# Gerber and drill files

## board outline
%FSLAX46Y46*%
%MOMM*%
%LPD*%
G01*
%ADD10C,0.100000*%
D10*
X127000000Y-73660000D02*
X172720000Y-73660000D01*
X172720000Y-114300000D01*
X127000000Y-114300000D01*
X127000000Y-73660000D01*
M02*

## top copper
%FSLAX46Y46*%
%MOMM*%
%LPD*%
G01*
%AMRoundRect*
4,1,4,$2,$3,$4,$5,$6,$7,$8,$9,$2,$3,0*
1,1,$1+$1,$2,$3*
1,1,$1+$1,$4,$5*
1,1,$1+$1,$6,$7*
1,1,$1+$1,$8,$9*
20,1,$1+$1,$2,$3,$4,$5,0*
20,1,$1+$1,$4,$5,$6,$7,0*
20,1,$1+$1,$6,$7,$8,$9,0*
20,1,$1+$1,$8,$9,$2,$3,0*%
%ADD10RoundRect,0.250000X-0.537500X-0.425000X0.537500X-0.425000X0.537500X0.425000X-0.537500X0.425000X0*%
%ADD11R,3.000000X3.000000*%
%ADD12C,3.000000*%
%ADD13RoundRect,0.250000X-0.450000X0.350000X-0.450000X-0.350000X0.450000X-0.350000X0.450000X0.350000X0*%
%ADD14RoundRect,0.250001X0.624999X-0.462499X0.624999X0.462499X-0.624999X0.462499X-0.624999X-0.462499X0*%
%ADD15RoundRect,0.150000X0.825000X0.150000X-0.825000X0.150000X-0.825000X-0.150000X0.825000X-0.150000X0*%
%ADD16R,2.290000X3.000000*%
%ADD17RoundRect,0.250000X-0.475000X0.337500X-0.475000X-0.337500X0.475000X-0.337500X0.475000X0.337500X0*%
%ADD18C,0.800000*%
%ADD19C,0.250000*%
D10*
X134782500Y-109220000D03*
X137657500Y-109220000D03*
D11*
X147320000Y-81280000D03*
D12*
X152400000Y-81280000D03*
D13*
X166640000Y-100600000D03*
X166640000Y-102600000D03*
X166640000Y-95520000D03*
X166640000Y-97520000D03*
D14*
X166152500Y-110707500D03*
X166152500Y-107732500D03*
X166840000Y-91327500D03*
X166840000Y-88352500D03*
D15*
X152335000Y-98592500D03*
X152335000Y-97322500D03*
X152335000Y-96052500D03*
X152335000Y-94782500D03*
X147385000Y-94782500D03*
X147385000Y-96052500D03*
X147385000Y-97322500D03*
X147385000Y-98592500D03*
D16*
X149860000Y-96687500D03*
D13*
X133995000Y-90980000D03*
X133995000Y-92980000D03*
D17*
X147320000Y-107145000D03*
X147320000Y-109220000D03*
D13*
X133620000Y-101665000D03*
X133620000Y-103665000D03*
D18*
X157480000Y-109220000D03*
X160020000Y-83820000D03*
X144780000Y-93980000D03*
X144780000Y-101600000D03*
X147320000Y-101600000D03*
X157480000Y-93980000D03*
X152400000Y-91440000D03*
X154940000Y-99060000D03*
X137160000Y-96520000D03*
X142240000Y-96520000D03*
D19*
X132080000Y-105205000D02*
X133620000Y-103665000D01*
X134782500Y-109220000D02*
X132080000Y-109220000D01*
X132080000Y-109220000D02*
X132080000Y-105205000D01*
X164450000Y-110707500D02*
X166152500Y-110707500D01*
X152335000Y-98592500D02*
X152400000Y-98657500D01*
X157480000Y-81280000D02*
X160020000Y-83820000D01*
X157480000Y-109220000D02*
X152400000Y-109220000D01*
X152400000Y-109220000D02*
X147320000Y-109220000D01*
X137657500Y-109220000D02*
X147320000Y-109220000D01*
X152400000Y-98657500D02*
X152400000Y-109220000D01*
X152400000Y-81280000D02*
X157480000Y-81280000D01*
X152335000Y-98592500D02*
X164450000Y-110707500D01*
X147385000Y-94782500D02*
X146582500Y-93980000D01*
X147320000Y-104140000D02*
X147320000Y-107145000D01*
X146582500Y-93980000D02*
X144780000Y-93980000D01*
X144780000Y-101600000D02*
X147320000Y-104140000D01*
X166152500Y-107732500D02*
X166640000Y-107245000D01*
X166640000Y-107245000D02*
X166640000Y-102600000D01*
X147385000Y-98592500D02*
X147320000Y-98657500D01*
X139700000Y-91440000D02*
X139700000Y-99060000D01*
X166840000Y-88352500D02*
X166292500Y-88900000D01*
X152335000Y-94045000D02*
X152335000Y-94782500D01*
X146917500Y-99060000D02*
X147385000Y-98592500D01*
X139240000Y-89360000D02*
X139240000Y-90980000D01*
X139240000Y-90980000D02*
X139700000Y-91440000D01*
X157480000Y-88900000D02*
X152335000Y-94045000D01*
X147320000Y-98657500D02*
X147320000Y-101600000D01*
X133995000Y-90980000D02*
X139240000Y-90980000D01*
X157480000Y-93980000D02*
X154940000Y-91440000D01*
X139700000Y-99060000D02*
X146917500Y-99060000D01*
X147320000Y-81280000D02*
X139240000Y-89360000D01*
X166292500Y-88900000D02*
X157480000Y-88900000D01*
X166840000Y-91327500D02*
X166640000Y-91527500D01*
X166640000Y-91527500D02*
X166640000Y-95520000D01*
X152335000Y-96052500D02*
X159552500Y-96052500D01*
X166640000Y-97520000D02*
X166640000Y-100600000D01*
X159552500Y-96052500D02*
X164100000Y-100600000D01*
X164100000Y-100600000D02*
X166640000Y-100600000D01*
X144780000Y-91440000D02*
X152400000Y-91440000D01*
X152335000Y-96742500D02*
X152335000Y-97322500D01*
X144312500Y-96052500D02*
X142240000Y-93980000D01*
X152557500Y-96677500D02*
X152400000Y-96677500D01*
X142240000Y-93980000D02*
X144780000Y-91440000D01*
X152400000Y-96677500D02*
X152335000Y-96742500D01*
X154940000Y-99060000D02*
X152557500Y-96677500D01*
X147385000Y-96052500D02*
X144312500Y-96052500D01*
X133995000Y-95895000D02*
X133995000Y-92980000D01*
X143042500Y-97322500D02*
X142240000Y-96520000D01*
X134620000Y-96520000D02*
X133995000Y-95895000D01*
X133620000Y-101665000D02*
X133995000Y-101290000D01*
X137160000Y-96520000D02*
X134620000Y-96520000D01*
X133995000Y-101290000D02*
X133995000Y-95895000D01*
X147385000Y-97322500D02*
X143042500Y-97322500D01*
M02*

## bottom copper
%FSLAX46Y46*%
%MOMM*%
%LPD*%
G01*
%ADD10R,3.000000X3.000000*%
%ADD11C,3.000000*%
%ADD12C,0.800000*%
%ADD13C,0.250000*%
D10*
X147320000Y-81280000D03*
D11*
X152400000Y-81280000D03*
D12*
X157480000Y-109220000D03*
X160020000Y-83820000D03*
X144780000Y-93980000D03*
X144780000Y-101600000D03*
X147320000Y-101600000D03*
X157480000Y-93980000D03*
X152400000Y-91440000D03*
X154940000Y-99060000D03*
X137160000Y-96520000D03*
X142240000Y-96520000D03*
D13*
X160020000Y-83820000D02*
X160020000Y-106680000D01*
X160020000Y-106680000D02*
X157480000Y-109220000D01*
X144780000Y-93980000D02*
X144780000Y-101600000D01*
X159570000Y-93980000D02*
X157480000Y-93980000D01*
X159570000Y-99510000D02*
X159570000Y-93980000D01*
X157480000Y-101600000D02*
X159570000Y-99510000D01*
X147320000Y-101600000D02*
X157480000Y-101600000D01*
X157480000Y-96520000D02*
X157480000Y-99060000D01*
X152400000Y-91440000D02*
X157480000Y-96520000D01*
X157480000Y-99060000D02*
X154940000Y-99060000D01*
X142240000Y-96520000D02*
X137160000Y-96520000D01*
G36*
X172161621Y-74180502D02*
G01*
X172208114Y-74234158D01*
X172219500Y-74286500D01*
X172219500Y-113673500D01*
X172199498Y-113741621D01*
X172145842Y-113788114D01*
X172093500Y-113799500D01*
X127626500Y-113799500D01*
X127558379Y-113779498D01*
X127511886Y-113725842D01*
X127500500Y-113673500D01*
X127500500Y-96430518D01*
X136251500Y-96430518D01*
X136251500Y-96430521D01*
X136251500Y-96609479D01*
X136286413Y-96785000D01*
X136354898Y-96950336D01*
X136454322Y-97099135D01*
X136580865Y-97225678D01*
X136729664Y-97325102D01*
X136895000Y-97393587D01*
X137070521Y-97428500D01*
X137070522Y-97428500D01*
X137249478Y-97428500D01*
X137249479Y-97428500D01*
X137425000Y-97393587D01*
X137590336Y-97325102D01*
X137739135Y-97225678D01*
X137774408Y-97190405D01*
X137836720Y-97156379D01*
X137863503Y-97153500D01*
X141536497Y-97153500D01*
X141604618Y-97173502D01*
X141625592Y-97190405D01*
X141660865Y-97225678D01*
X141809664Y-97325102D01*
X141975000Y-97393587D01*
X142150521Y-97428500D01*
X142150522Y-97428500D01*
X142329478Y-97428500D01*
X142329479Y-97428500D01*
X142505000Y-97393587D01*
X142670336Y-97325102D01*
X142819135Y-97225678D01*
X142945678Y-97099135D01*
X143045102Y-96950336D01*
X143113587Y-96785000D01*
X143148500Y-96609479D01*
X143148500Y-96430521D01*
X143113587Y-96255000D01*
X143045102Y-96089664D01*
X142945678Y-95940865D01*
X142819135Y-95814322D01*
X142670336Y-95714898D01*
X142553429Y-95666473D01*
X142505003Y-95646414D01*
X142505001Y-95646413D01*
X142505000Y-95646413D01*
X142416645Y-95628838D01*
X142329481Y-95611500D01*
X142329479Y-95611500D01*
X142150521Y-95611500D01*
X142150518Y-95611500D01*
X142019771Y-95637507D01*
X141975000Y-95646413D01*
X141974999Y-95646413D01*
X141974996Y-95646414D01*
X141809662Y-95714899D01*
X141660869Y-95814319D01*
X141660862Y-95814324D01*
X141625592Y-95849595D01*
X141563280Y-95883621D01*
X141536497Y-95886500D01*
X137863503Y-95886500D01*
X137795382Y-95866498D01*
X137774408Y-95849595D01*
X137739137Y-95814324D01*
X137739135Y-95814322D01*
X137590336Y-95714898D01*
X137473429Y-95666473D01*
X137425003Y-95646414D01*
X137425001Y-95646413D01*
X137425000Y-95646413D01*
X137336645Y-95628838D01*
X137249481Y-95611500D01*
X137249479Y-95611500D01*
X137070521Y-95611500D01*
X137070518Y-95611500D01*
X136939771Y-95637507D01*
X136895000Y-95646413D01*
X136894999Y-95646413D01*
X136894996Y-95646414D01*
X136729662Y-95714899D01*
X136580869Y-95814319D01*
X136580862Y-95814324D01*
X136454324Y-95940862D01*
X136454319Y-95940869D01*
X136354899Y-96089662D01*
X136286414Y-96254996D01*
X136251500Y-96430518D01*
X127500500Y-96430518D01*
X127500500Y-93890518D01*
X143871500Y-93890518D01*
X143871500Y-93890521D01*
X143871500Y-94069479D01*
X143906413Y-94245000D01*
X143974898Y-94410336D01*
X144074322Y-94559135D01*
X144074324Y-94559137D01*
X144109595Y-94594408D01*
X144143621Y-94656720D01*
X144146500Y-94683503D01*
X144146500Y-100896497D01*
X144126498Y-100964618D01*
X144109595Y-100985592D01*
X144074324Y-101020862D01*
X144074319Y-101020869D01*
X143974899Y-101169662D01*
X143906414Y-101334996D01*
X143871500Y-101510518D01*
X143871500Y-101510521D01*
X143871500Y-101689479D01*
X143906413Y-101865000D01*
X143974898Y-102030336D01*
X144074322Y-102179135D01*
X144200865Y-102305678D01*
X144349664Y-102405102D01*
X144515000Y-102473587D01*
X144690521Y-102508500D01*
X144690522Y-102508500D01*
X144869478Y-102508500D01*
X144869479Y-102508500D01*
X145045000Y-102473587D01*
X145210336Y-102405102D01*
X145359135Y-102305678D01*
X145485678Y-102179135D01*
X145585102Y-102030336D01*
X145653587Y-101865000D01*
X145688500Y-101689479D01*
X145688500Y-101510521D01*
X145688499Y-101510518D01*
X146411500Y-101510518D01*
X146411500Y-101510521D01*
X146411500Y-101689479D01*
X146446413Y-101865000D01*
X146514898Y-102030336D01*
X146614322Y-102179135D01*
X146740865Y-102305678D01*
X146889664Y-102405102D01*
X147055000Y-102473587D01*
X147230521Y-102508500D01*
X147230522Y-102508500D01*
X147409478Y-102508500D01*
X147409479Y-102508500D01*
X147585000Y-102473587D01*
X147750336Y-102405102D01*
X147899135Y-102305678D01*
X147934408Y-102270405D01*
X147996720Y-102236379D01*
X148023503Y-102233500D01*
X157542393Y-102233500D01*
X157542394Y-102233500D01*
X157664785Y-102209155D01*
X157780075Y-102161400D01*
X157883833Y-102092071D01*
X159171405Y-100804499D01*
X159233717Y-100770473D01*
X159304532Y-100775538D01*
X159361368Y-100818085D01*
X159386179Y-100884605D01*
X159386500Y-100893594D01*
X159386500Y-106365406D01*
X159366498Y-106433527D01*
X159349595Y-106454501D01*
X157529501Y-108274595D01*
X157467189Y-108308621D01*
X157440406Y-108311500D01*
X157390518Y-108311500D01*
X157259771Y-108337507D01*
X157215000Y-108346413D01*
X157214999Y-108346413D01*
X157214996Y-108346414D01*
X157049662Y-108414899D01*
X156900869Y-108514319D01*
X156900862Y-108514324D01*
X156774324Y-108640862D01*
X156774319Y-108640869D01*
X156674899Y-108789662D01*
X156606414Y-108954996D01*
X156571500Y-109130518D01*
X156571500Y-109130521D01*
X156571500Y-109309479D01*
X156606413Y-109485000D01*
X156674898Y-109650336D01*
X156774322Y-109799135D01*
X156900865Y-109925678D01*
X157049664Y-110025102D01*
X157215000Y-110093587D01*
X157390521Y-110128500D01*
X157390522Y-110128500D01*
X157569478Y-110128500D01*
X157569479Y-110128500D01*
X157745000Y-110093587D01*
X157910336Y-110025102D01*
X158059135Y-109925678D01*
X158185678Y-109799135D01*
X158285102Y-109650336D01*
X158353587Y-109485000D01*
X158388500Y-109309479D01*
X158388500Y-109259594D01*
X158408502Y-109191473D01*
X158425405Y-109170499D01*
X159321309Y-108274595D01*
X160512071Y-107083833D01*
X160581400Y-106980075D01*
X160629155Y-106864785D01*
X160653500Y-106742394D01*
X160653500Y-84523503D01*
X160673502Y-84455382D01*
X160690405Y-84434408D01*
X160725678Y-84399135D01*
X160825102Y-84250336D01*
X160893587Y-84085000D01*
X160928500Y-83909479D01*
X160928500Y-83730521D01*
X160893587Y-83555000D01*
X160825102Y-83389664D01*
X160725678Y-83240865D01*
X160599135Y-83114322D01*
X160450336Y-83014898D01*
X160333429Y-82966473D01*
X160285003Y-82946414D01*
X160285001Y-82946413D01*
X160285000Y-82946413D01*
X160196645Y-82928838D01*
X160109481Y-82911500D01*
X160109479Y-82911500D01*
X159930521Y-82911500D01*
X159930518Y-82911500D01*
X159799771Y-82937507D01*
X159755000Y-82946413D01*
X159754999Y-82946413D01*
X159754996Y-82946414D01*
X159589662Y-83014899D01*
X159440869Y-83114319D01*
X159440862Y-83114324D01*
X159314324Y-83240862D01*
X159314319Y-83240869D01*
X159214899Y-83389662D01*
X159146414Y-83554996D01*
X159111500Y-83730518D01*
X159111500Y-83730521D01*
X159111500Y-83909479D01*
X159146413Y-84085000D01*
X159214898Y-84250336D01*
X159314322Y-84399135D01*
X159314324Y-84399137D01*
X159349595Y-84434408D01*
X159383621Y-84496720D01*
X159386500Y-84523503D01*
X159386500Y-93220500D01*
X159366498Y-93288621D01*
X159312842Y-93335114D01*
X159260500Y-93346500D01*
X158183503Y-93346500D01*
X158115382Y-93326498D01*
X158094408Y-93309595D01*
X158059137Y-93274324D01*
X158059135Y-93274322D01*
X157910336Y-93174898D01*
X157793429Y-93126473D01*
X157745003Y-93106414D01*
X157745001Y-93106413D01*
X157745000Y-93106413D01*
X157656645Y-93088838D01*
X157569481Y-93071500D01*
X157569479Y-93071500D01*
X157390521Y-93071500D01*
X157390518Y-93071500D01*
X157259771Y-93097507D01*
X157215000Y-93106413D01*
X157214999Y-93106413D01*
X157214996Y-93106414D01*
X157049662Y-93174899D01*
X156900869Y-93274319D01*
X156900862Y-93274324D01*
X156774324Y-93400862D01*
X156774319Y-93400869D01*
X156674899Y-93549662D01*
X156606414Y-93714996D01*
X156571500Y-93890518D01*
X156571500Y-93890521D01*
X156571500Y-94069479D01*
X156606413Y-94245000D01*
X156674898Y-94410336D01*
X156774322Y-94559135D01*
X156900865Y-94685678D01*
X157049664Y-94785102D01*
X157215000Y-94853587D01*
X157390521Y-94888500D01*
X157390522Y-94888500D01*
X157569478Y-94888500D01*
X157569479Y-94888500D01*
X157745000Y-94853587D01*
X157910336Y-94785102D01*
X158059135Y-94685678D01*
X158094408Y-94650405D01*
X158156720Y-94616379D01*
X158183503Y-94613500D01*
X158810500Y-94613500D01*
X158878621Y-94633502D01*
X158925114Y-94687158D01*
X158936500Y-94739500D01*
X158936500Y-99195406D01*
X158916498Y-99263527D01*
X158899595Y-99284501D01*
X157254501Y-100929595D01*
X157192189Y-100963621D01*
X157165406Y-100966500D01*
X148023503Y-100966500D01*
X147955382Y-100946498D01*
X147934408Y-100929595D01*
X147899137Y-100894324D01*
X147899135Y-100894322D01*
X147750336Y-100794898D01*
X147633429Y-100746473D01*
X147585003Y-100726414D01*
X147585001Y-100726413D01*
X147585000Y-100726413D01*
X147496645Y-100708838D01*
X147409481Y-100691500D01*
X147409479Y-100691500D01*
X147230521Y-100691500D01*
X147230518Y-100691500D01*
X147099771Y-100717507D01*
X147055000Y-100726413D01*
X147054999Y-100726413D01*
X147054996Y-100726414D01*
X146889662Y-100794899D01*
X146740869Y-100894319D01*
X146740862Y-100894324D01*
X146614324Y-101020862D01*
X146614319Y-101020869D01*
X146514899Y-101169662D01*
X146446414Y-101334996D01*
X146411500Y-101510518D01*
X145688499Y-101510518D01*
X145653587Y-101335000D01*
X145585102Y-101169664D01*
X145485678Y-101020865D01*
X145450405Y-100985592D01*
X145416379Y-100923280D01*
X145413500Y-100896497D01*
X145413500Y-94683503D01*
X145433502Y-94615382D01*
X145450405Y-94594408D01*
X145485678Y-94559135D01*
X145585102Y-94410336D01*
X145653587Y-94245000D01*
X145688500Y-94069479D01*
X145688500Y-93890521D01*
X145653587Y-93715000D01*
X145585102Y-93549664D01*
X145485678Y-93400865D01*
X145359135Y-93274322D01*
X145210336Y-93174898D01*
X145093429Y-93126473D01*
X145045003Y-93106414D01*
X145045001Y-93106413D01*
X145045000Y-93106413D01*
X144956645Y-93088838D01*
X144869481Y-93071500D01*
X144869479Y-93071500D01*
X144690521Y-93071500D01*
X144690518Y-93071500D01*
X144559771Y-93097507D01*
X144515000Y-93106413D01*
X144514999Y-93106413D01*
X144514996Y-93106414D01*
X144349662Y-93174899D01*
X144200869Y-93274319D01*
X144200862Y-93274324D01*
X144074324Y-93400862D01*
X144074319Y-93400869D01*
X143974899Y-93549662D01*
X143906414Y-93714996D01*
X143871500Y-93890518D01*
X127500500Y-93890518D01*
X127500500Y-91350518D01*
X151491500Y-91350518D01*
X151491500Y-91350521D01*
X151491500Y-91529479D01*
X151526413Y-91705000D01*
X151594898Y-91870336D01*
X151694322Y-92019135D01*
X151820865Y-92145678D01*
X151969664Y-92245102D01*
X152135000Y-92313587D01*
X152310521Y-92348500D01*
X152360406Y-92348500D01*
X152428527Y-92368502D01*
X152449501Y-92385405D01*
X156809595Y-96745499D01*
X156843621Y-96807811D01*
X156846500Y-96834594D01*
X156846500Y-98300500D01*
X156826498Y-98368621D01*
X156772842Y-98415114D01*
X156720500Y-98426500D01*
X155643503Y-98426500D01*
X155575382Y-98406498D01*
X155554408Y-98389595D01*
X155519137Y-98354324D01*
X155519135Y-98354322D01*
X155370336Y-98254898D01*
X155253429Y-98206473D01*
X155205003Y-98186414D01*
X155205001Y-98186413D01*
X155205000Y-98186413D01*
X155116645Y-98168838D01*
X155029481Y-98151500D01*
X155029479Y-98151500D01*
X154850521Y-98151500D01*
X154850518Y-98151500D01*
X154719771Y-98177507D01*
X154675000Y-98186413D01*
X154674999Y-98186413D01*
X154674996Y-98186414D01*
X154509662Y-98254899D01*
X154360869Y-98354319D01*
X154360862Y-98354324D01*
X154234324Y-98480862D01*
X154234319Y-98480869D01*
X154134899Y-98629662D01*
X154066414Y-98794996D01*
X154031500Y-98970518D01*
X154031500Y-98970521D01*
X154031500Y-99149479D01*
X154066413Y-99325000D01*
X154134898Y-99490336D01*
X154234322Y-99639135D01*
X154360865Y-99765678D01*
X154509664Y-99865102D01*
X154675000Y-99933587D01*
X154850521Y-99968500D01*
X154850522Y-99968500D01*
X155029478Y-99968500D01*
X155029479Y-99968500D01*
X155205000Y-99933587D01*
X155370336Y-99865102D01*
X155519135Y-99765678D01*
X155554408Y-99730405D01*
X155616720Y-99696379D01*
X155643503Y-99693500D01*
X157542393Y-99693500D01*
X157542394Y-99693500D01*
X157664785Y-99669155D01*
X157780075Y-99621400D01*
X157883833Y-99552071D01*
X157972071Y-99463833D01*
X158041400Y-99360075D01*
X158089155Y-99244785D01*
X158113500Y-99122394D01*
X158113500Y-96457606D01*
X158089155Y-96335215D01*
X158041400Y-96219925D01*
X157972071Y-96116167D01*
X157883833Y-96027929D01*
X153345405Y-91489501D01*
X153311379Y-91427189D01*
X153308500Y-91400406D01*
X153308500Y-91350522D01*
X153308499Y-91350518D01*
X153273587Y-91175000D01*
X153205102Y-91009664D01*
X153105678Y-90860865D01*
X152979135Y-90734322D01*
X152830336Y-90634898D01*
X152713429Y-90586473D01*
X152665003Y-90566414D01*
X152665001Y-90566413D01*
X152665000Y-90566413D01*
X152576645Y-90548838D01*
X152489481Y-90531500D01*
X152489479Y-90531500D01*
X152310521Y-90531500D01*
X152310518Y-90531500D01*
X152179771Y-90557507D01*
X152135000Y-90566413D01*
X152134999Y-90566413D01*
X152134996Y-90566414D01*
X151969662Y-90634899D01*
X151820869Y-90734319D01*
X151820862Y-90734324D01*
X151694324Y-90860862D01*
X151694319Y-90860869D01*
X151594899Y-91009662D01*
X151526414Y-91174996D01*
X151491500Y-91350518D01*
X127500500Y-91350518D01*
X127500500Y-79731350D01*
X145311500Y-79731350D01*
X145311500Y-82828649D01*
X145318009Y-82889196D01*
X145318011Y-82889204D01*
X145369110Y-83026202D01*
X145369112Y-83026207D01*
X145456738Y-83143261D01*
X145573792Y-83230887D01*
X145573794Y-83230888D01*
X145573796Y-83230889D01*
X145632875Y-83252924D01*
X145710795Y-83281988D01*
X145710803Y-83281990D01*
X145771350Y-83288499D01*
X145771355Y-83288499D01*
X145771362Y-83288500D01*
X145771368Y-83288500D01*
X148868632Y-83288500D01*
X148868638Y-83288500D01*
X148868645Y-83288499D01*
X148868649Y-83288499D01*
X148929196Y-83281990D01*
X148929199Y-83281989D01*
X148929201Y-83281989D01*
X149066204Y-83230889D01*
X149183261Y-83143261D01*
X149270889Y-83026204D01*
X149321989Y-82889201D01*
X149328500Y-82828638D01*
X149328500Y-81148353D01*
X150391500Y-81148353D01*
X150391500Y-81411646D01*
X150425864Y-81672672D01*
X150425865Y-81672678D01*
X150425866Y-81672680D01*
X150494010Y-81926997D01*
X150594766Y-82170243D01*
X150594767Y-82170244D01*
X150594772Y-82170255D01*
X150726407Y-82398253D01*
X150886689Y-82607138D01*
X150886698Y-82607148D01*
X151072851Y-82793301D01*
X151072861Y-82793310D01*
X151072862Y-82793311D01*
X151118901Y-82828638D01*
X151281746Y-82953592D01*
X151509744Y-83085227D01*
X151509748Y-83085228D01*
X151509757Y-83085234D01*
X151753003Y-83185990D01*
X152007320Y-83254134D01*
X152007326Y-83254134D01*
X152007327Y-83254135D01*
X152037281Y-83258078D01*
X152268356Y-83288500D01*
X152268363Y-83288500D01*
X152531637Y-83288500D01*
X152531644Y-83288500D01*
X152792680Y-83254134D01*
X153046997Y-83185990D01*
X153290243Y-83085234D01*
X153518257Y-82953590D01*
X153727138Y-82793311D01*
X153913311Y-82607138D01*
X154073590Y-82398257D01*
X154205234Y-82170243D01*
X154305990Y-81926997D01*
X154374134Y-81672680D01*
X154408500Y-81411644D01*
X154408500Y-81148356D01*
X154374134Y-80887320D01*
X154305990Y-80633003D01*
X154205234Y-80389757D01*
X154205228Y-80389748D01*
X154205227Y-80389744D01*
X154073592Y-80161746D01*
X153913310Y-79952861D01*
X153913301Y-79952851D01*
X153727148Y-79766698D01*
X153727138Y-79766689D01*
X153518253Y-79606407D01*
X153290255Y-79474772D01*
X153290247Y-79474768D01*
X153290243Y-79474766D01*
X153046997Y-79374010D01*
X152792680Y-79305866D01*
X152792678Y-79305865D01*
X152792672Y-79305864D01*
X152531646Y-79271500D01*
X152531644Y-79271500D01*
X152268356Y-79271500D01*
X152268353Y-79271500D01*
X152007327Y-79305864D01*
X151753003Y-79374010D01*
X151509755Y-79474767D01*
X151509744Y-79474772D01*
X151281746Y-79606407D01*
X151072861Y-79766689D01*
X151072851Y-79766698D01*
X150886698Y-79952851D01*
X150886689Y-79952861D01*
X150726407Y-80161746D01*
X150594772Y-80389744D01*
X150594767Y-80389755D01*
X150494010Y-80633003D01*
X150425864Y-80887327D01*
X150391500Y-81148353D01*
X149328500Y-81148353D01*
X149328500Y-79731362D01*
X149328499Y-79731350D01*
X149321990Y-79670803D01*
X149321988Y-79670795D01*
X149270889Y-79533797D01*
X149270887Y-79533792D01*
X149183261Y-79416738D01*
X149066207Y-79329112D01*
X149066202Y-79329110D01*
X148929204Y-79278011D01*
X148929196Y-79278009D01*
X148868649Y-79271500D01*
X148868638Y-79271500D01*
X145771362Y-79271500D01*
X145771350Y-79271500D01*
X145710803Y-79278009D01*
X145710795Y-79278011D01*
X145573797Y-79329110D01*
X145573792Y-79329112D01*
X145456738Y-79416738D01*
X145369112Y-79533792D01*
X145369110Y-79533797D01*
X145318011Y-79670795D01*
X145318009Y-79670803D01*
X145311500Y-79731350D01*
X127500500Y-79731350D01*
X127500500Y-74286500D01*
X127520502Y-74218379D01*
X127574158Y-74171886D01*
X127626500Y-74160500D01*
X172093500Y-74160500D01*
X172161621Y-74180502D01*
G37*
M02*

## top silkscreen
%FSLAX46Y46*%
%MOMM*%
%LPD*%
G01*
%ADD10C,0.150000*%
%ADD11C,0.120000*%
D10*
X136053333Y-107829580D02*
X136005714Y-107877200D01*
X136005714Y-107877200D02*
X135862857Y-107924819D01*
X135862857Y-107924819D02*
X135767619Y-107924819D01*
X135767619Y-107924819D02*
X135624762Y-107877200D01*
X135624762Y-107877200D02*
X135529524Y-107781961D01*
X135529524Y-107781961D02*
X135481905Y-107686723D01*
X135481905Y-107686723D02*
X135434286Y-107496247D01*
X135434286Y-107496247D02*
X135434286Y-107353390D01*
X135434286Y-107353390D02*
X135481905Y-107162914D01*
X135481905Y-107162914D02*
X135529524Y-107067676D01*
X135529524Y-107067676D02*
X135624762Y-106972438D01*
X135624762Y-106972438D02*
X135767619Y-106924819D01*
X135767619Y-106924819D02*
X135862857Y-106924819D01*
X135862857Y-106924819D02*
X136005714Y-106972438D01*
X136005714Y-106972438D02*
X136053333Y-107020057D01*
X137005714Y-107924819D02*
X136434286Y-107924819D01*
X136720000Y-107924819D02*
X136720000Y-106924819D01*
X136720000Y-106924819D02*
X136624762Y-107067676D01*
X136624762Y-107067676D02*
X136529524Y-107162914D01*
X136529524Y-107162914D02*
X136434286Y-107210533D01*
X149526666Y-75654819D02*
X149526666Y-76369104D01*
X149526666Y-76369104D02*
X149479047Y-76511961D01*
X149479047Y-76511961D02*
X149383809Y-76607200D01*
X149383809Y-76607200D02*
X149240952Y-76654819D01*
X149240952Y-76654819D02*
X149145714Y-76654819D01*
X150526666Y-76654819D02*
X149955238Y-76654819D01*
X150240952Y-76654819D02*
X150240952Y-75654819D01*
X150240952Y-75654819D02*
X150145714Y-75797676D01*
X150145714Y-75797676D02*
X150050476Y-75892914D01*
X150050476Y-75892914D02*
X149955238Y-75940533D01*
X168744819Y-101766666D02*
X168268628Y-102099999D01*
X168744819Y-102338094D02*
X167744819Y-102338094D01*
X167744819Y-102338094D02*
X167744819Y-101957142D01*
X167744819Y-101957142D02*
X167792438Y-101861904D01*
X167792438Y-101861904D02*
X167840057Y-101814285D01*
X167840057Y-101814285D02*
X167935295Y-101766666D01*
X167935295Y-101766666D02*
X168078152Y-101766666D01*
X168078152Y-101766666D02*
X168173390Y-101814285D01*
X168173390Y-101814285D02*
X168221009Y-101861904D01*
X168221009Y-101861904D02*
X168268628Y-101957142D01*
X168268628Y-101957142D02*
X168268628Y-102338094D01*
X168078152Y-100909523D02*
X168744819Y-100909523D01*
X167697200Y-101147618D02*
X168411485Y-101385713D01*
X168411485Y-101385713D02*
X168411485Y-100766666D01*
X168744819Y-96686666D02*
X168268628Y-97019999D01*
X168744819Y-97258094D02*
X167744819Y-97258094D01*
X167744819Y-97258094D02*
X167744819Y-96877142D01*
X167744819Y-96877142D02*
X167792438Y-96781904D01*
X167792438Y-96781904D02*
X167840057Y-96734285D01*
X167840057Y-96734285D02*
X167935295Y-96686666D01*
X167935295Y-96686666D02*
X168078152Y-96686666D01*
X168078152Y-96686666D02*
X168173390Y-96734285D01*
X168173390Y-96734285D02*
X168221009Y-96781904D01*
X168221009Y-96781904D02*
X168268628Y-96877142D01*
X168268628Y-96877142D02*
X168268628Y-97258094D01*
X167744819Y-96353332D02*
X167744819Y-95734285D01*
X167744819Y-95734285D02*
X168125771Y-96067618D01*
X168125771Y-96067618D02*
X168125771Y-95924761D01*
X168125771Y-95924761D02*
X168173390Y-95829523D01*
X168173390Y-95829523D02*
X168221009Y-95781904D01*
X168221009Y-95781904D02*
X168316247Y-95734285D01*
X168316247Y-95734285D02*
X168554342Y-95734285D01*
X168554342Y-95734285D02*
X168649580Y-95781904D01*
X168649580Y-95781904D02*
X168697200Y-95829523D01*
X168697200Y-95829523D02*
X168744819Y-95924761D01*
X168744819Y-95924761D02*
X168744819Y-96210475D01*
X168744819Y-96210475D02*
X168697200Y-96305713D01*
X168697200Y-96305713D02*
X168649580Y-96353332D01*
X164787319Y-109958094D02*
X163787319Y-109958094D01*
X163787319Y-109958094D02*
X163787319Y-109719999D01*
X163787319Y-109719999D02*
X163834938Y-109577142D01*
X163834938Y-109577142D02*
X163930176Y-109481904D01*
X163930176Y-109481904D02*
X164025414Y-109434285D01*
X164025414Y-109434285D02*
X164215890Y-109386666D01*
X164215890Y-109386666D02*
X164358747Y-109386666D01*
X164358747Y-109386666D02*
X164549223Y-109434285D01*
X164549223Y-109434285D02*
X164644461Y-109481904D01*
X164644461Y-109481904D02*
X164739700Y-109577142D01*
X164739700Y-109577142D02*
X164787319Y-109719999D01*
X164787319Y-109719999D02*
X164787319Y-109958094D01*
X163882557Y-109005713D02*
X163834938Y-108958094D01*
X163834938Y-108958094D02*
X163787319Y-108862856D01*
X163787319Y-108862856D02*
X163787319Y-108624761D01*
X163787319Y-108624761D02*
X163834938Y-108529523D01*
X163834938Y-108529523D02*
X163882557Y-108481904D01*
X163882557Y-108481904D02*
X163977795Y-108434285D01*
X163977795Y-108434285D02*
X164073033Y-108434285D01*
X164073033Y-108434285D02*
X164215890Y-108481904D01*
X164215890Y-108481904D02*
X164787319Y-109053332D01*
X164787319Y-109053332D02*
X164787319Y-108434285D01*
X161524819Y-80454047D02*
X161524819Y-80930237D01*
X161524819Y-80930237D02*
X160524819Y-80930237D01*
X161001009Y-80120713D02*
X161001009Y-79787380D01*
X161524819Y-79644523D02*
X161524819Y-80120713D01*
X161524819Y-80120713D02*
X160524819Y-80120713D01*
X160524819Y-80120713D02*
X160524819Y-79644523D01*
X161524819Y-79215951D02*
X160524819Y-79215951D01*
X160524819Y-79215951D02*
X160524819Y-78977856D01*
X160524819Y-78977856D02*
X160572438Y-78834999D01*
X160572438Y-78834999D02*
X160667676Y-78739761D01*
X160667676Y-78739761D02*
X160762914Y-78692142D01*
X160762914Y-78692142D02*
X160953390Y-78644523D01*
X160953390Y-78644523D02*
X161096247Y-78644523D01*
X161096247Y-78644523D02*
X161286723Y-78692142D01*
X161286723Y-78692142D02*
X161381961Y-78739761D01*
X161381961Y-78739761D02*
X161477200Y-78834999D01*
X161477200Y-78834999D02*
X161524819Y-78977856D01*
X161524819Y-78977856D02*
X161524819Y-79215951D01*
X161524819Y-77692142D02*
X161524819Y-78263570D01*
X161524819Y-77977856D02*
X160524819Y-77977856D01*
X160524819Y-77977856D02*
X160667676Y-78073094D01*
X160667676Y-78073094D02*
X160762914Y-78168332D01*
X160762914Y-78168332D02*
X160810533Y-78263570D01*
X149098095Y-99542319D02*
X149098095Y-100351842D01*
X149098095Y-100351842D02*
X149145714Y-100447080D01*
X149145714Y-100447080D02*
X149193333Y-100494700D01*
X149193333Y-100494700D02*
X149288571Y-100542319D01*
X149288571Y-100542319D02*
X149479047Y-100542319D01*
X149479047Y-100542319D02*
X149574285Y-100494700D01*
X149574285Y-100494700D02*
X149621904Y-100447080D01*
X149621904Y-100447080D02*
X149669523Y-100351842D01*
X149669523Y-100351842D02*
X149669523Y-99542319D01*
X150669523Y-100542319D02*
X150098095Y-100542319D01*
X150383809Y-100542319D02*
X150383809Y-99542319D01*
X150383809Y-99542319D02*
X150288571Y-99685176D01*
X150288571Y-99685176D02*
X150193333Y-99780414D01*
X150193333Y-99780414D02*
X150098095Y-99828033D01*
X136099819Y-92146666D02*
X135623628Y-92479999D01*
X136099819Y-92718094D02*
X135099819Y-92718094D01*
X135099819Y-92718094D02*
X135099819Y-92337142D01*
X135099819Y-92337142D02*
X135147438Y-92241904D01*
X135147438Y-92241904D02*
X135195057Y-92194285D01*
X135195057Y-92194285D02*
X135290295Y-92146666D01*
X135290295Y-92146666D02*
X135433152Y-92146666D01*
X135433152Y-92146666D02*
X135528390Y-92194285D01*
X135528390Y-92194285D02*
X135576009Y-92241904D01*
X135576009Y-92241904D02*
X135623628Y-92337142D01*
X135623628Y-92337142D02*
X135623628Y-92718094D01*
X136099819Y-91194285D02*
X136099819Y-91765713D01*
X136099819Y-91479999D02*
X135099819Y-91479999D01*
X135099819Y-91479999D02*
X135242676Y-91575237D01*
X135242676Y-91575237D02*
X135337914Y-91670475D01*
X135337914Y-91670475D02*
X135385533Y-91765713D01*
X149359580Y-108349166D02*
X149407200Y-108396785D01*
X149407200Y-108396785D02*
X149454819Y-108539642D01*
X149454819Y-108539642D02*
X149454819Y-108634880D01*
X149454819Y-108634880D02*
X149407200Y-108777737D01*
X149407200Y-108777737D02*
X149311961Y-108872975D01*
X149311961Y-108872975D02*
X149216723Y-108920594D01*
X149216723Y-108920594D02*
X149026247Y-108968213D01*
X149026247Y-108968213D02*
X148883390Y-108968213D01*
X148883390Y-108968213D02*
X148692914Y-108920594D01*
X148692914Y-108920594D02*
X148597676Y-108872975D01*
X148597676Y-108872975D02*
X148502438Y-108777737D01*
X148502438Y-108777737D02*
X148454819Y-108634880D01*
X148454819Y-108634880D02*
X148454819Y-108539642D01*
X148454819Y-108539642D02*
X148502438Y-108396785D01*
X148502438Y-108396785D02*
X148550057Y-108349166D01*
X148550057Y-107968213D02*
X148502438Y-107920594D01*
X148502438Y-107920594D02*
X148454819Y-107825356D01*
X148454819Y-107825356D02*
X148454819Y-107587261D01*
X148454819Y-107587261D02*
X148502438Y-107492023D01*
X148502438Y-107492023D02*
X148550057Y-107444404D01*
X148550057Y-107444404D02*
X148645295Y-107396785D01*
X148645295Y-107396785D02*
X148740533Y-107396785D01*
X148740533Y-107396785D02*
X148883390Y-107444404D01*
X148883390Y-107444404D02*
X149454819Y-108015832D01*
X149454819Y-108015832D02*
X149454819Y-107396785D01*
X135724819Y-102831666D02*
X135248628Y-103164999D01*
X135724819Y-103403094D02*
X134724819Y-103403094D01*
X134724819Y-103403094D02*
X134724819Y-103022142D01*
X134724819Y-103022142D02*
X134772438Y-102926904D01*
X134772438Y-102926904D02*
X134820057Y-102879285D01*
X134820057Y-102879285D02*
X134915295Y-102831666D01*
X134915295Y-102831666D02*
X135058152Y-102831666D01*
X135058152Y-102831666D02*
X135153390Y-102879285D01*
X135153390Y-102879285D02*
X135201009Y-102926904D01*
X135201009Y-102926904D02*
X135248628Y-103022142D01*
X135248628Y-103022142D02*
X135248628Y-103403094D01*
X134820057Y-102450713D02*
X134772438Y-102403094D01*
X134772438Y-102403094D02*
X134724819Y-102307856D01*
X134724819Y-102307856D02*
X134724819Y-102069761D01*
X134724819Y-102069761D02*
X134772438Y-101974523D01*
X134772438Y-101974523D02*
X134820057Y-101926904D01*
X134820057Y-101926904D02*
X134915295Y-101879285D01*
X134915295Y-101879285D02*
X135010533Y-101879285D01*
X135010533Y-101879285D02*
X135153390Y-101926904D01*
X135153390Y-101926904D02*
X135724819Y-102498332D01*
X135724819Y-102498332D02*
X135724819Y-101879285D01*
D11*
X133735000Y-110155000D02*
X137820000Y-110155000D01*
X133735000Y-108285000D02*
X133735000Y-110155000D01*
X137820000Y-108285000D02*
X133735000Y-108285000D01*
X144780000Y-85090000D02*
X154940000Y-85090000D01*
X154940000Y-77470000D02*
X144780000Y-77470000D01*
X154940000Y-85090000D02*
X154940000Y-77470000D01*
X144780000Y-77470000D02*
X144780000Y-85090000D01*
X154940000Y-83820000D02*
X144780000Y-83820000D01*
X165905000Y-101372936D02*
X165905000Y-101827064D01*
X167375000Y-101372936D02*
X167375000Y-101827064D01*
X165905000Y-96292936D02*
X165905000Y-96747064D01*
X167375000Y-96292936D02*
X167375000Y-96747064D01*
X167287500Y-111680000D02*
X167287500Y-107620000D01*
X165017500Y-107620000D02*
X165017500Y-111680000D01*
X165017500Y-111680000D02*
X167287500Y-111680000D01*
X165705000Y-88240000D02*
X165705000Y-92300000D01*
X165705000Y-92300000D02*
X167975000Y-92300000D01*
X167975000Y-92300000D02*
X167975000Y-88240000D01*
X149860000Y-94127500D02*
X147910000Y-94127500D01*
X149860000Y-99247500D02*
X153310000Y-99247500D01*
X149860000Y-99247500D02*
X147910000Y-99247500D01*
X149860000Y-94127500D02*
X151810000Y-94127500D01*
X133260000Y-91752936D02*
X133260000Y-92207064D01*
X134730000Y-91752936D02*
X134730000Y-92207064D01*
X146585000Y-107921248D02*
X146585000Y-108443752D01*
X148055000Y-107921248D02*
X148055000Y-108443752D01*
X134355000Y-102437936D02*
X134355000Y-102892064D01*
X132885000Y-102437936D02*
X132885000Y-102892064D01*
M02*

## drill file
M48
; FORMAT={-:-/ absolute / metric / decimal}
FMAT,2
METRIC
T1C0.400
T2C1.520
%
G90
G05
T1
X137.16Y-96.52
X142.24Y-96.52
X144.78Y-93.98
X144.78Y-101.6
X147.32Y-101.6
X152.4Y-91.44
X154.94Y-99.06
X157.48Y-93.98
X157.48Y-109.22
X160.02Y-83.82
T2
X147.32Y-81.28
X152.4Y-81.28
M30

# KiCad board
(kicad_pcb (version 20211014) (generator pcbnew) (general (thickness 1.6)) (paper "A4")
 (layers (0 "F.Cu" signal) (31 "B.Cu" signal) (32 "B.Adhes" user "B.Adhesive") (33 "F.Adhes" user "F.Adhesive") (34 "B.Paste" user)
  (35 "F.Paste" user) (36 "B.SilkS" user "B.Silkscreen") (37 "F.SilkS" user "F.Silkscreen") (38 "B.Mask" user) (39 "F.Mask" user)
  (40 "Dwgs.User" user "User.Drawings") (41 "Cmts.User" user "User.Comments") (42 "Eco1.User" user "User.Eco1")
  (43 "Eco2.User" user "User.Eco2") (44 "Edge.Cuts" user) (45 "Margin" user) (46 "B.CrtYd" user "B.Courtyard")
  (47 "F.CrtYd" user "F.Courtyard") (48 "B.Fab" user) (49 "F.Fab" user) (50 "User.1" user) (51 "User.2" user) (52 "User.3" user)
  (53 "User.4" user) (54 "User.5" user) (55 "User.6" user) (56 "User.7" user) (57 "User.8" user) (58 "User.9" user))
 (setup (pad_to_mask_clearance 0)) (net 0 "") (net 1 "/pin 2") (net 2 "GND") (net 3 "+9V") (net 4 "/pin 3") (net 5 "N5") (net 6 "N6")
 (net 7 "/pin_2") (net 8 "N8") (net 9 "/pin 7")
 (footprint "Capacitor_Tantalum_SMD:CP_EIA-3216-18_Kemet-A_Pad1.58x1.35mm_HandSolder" (layer "F.Cu") (at 136.22 109.22)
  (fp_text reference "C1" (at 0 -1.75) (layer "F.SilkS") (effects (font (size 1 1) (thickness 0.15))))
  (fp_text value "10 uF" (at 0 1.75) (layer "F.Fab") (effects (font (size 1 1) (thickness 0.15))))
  (fp_line (start -2.485 0.935) (end 1.6 0.935) (layer "F.SilkS") (width 0.12))
  (fp_line (start -2.485 -0.935) (end -2.485 0.935) (layer "F.SilkS") (width 0.12))
  (fp_line (start 1.6 -0.935) (end -2.485 -0.935) (layer "F.SilkS") (width 0.12))
  (pad "1" smd roundrect (at -1.4375 0) (size 1.575 1.35) (layers "F.Cu" "F.Paste" "F.Mask") (roundrect_rratio 0.1851851852)
   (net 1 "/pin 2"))
  (pad "2" smd roundrect (at 1.4375 0) (size 1.575 1.35) (layers "F.Cu" "F.Paste" "F.Mask") (roundrect_rratio 0.1851851852) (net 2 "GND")))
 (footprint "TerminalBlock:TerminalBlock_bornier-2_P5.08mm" (layer "F.Cu") (at 147.32 81.28)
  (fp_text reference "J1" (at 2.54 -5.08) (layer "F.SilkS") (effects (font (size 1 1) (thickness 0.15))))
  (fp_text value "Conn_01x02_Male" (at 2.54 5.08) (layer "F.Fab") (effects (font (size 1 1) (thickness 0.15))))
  (fp_line (start -2.54 3.81) (end 7.62 3.81) (layer "F.SilkS") (width 0.12))
  (fp_line (start 7.62 -3.81) (end -2.54 -3.81) (layer "F.SilkS") (width 0.12))
  (fp_line (start 7.62 3.81) (end 7.62 -3.81) (layer "F.SilkS") (width 0.12))
  (fp_line (start -2.54 -3.81) (end -2.54 3.81) (layer "F.SilkS") (width 0.12))
  (fp_line (start 7.62 2.54) (end -2.54 2.54) (layer "F.SilkS") (width 0.12))
  (pad "1" thru_hole rect (at 0 0) (size 3 3) (drill 1.52) (layers *.Cu *.Mask) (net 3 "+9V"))
  (pad "2" thru_hole circle (at 5.08 0) (size 3 3) (drill 1.52) (layers *.Cu *.Mask) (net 2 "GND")))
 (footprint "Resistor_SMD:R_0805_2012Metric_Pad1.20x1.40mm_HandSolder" (layer "F.Cu") (at 166.64 101.6 -90)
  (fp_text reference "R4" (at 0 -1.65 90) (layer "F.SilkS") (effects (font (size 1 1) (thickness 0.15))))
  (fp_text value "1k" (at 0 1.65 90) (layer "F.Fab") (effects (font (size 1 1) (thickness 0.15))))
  (fp_line (start -0.227064 0.735) (end 0.227064 0.735) (layer "F.SilkS") (width 0.12))
  (fp_line (start -0.227064 -0.735) (end 0.227064 -0.735) (layer "F.SilkS") (width 0.12))
  (pad "1" smd roundrect (at -1 0 270) (size 1.2 1.4) (layers "F.Cu" "F.Paste" "F.Mask") (roundrect_rratio 0.2083333333) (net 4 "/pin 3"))
  (pad "2" smd roundrect (at 1 0 270) (size 1.2 1.4) (layers "F.Cu" "F.Paste" "F.Mask") (roundrect_rratio 0.2083333333) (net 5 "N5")))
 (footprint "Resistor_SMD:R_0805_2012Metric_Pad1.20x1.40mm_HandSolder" (layer "F.Cu") (at 166.64 96.52 -90)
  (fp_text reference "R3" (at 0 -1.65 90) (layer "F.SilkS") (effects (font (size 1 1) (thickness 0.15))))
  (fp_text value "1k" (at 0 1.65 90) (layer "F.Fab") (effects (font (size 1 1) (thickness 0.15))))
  (fp_line (start -0.227064 0.735) (end 0.227064 0.735) (layer "F.SilkS") (width 0.12))
  (fp_line (start -0.227064 -0.735) (end 0.227064 -0.735) (layer "F.SilkS") (width 0.12))
  (pad "1" smd roundrect (at -1 0 270) (size 1.2 1.4) (layers "F.Cu" "F.Paste" "F.Mask") (roundrect_rratio 0.2083333333) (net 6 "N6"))
  (pad "2" smd roundrect (at 1 0 270) (size 1.2 1.4) (layers "F.Cu" "F.Paste" "F.Mask") (roundrect_rratio 0.2083333333) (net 4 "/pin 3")))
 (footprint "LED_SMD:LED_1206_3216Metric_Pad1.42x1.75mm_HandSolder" (layer "F.Cu") (at 166.1525 109.22 90)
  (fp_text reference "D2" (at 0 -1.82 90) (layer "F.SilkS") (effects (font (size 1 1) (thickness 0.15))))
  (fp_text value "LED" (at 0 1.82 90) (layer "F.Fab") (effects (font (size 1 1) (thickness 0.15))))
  (fp_line (start -2.46 1.135) (end 1.6 1.135) (layer "F.SilkS") (width 0.12))
  (fp_line (start 1.6 -1.135) (end -2.46 -1.135) (layer "F.SilkS") (width 0.12))
  (fp_line (start -2.46 -1.135) (end -2.46 1.135) (layer "F.SilkS") (width 0.12))
  (pad "1" smd roundrect (at -1.4875 0 90) (size 1.425 1.75) (layers "F.Cu" "F.Paste" "F.Mask") (roundrect_rratio 0.1754392982)
   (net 2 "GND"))
  (pad "2" smd roundrect (at 1.4875 0 90) (size 1.425 1.75) (layers "F.Cu" "F.Paste" "F.Mask") (roundrect_rratio 0.1754392982) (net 5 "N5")))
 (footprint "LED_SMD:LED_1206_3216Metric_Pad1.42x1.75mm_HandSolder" (layer "F.Cu") (at 166.84 89.84 90)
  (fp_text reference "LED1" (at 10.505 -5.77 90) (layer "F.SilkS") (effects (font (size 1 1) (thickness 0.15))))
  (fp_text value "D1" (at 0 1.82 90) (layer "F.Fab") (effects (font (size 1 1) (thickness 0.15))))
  (fp_line (start 1.6 -1.135) (end -2.46 -1.135) (layer "F.SilkS") (width 0.12))
  (fp_line (start -2.46 -1.135) (end -2.46 1.135) (layer "F.SilkS") (width 0.12))
  (fp_line (start -2.46 1.135) (end 1.6 1.135) (layer "F.SilkS") (width 0.12))
  (pad "1" smd roundrect (at -1.4875 0 90) (size 1.425 1.75) (layers "F.Cu" "F.Paste" "F.Mask") (roundrect_rratio 0.1754392982) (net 6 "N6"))
  (pad "2" smd roundrect (at 1.4875 0 90) (size 1.425 1.75) (layers "F.Cu" "F.Paste" "F.Mask") (roundrect_rratio 0.1754392982) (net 3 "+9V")))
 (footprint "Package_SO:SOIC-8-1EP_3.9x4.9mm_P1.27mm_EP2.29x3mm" (layer "F.Cu") (at 149.86 96.6875 180)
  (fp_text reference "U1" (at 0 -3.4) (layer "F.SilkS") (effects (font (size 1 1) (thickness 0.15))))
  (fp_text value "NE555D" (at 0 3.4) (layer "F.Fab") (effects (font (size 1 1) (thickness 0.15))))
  (fp_line (start 0 2.56) (end 1.95 2.56) (layer "F.SilkS") (width 0.12))
  (fp_line (start 0 -2.56) (end -3.45 -2.56) (layer "F.SilkS") (width 0.12))
  (fp_line (start 0 -2.56) (end 1.95 -2.56) (layer "F.SilkS") (width 0.12))
  (fp_line (start 0 2.56) (end -1.95 2.56) (layer "F.SilkS") (width 0.12))
  (pad "" smd roundrect (at -0.57 0.75 180) (size 0.92 1.21) (layers "F.Paste") (roundrect_rratio 0.25))
  (pad "" smd roundrect (at 0.57 -0.75 180) (size 0.92 1.21) (layers "F.Paste") (roundrect_rratio 0.25))
  (pad "" smd roundrect (at 0.57 0.75 180) (size 0.92 1.21) (layers "F.Paste") (roundrect_rratio 0.25))
  (pad "" smd roundrect (at -0.57 -0.75 180) (size 0.92 1.21) (layers "F.Paste") (roundrect_rratio 0.25))
  (pad "1" smd roundrect (at -2.475 -1.905 180) (size 1.95 0.6) (layers "F.Cu" "F.Paste" "F.Mask") (roundrect_rratio 0.25) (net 2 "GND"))
  (pad "2" smd roundrect (at -2.475 -0.635 180) (size 1.95 0.6) (layers "F.Cu" "F.Paste" "F.Mask") (roundrect_rratio 0.25) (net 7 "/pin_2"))
  (pad "3" smd roundrect (at -2.475 0.635 180) (size 1.95 0.6) (layers "F.Cu" "F.Paste" "F.Mask") (roundrect_rratio 0.25) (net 4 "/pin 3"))
  (pad "4" smd roundrect (at -2.475 1.905 180) (size 1.95 0.6) (layers "F.Cu" "F.Paste" "F.Mask") (roundrect_rratio 0.25) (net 3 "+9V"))
  (pad "5" smd roundrect (at 2.475 1.905 180) (size 1.95 0.6) (layers "F.Cu" "F.Paste" "F.Mask") (roundrect_rratio 0.25) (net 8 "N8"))
  (pad "6" smd roundrect (at 2.475 0.635 180) (size 1.95 0.6) (layers "F.Cu" "F.Paste" "F.Mask") (roundrect_rratio 0.25) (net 7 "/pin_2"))
  (pad "7" smd roundrect (at 2.475 -0.635 180) (size 1.95 0.6) (layers "F.Cu" "F.Paste" "F.Mask") (roundrect_rratio 0.25) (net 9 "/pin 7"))
  (pad "8" smd roundrect (at 2.475 -1.905 180) (size 1.95 0.6) (layers "F.Cu" "F.Paste" "F.Mask") (roundrect_rratio 0.25) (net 3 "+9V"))
  (pad "9" smd rect (at 0 0 180) (size 2.29 3) (layers "F.Cu" "F.Mask")))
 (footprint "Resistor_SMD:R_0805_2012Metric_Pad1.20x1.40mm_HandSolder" (layer "F.Cu") (at 133.995 91.98 -90)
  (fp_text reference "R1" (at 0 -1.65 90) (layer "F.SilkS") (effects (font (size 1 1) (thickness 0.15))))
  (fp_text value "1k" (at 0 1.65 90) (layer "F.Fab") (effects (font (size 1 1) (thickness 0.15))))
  (fp_line (start -0.227064 0.735) (end 0.227064 0.735) (layer "F.SilkS") (width 0.12))
  (fp_line (start -0.227064 -0.735) (end 0.227064 -0.735) (layer "F.SilkS") (width 0.12))
  (pad "1" smd roundrect (at -1 0 270) (size 1.2 1.4) (layers "F.Cu" "F.Paste" "F.Mask") (roundrect_rratio 0.2083333333) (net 3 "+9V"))
  (pad "2" smd roundrect (at 1 0 270) (size 1.2 1.4) (layers "F.Cu" "F.Paste" "F.Mask") (roundrect_rratio 0.2083333333) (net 9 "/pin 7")))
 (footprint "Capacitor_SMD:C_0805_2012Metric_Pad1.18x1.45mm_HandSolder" (layer "F.Cu") (at 147.32 108.1825 -90)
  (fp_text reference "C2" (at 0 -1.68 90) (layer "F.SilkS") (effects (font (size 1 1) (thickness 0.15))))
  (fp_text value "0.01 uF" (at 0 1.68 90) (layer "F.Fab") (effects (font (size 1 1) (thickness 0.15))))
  (fp_line (start -0.261252 0.735) (end 0.261252 0.735) (layer "F.SilkS") (width 0.12))
  (fp_line (start -0.261252 -0.735) (end 0.261252 -0.735) (layer "F.SilkS") (width 0.12))
  (pad "1" smd roundrect (at -1.0375 0 270) (size 1.175 1.45) (layers "F.Cu" "F.Paste" "F.Mask") (roundrect_rratio 0.2127659574)
   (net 8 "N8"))
  (pad "2" smd roundrect (at 1.0375 0 270) (size 1.175 1.45) (layers "F.Cu" "F.Paste" "F.Mask") (roundrect_rratio 0.2127659574)
   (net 2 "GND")))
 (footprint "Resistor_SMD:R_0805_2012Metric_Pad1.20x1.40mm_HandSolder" (layer "F.Cu") (at 133.62 102.665 -90)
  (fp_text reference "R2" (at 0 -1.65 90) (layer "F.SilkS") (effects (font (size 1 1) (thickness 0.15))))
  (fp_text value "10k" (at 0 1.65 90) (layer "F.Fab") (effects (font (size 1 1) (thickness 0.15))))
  (fp_line (start -0.227064 -0.735) (end 0.227064 -0.735) (layer "F.SilkS") (width 0.12))
  (fp_line (start -0.227064 0.735) (end 0.227064 0.735) (layer "F.SilkS") (width 0.12))
  (pad "1" smd roundrect (at -1 0 270) (size 1.2 1.4) (layers "F.Cu" "F.Paste" "F.Mask") (roundrect_rratio 0.2083333333) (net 9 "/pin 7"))
  (pad "2" smd roundrect (at 1 0 270) (size 1.2 1.4) (layers "F.Cu" "F.Paste" "F.Mask") (roundrect_rratio 0.2083333333) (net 1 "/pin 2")))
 (gr_rect (start 127 73.66) (end 172.72 114.3) (layer "Edge.Cuts") (width 0.1) (fill none))
 (segment (start 132.08 105.205) (end 133.62 103.665) (width 0.25) (layer "F.Cu") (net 1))
 (segment (start 134.7825 109.22) (end 132.08 109.22) (width 0.25) (layer "F.Cu") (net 1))
 (segment (start 132.08 109.22) (end 132.08 105.205) (width 0.25) (layer "F.Cu") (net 1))
 (segment (start 164.45 110.7075) (end 166.1525 110.7075) (width 0.25) (layer "F.Cu") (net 2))
 (segment (start 152.335 98.5925) (end 152.4 98.6575) (width 0.25) (layer "F.Cu") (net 2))
 (segment (start 157.48 81.28) (end 160.02 83.82) (width 0.25) (layer "F.Cu") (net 2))
 (segment (start 157.48 109.22) (end 152.4 109.22) (width 0.25) (layer "F.Cu") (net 2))
 (segment (start 152.4 109.22) (end 147.32 109.22) (width 0.25) (layer "F.Cu") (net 2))
 (segment (start 137.6575 109.22) (end 147.32 109.22) (width 0.25) (layer "F.Cu") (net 2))
 (segment (start 152.4 98.6575) (end 152.4 109.22) (width 0.25) (layer "F.Cu") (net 2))
 (segment (start 152.4 81.28) (end 157.48 81.28) (width 0.25) (layer "F.Cu") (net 2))
 (segment (start 152.335 98.5925) (end 164.45 110.7075) (width 0.25) (layer "F.Cu") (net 2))
 (via (at 157.48 109.22) (size 0.8) (drill 0.4) (layers "F.Cu" "B.Cu") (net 2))
 (via (at 160.02 83.82) (size 0.8) (drill 0.4) (layers "F.Cu" "B.Cu") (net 2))
 (segment (start 160.02 83.82) (end 160.02 106.68) (width 0.25) (layer "B.Cu") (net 2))
 (segment (start 160.02 106.68) (end 157.48 109.22) (width 0.25) (layer "B.Cu") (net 2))
 (segment (start 147.385 94.7825) (end 146.5825 93.98) (width 0.25) (layer "F.Cu") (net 8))
 (segment (start 147.32 104.14) (end 147.32 107.145) (width 0.25) (layer "F.Cu") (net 8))
 (segment (start 146.5825 93.98) (end 144.78 93.98) (width 0.25) (layer "F.Cu") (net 8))
 (segment (start 144.78 101.6) (end 147.32 104.14) (width 0.25) (layer "F.Cu") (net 8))
 (via (at 144.78 93.98) (size 0.8) (drill 0.4) (layers "F.Cu" "B.Cu") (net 8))
 (via (at 144.78 101.6) (size 0.8) (drill 0.4) (layers "F.Cu" "B.Cu") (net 8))
 (segment (start 144.78 93.98) (end 144.78 101.6) (width 0.25) (layer "B.Cu") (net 8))
 (segment (start 166.1525 107.7325) (end 166.64 107.245) (width 0.25) (layer "F.Cu") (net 5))
 (segment (start 166.64 107.245) (end 166.64 102.6) (width 0.25) (layer "F.Cu") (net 5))
 (segment (start 147.385 98.5925) (end 147.32 98.6575) (width 0.25) (layer "F.Cu") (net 3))
 (segment (start 139.7 91.44) (end 139.7 99.06) (width 0.25) (layer "F.Cu") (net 3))
 (segment (start 166.84 88.3525) (end 166.2925 88.9) (width 0.25) (layer "F.Cu") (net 3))
 (segment (start 152.335 94.045) (end 152.335 94.7825) (width 0.25) (layer "F.Cu") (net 3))
 (segment (start 146.9175 99.06) (end 147.385 98.5925) (width 0.25) (layer "F.Cu") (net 3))
 (segment (start 139.24 89.36) (end 139.24 90.98) (width 0.25) (layer "F.Cu") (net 3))
 (segment (start 139.24 90.98) (end 139.7 91.44) (width 0.25) (layer "F.Cu") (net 3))
 (segment (start 157.48 88.9) (end 152.335 94.045) (width 0.25) (layer "F.Cu") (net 3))
 (segment (start 147.32 98.6575) (end 147.32 101.6) (width 0.25) (layer "F.Cu") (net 3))
 (segment (start 133.995 90.98) (end 139.24 90.98) (width 0.25) (layer "F.Cu") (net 3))
 (segment (start 157.48 93.98) (end 154.94 91.44) (width 0.25) (layer "F.Cu") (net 3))
 (segment (start 139.7 99.06) (end 146.9175 99.06) (width 0.25) (layer "F.Cu") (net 3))
 (segment (start 147.32 81.28) (end 139.24 89.36) (width 0.25) (layer "F.Cu") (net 3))
 (segment (start 166.2925 88.9) (end 157.48 88.9) (width 0.25) (layer "F.Cu") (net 3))
 (via (at 147.32 101.6) (size 0.8) (drill 0.4) (layers "F.Cu" "B.Cu") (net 3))
 (via (at 157.48 93.98) (size 0.8) (drill 0.4) (layers "F.Cu" "B.Cu") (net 3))
 (segment (start 159.57 93.98) (end 157.48 93.98) (width 0.25) (layer "B.Cu") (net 3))
 (segment (start 159.57 99.51) (end 159.57 93.98) (width 0.25) (layer "B.Cu") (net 3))
 (segment (start 157.48 101.6) (end 159.57 99.51) (width 0.25) (layer "B.Cu") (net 3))
 (segment (start 147.32 101.6) (end 157.48 101.6) (width 0.25) (layer "B.Cu") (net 3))
 (segment (start 166.84 91.3275) (end 166.64 91.5275) (width 0.25) (layer "F.Cu") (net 6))
 (segment (start 166.64 91.5275) (end 166.64 95.52) (width 0.25) (layer "F.Cu") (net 6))
 (segment (start 152.335 96.0525) (end 159.5525 96.0525) (width 0.25) (layer "F.Cu") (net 4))
 (segment (start 166.64 97.52) (end 166.64 100.6) (width 0.25) (layer "F.Cu") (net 4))
 (segment (start 159.5525 96.0525) (end 164.1 100.6) (width 0.25) (layer "F.Cu") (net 4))
 (segment (start 164.1 100.6) (end 166.64 100.6) (width 0.25) (layer "F.Cu") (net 4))
 (segment (start 144.78 91.44) (end 152.4 91.44) (width 0.25) (layer "F.Cu") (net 7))
 (segment (start 152.335 96.7425) (end 152.335 97.3225) (width 0.25) (layer "F.Cu") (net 7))
 (segment (start 144.3125 96.0525) (end 142.24 93.98) (width 0.25) (layer "F.Cu") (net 7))
 (segment (start 152.5575 96.6775) (end 152.4 96.6775) (width 0.25) (layer "F.Cu") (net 7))
 (segment (start 142.24 93.98) (end 144.78 91.44) (width 0.25) (layer "F.Cu") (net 7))
 (segment (start 152.4 96.6775) (end 152.335 96.7425) (width 0.25) (layer "F.Cu") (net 7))
 (segment (start 154.94 99.06) (end 152.5575 96.6775) (width 0.25) (layer "F.Cu") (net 7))
 (segment (start 147.385 96.0525) (end 144.3125 96.0525) (width 0.25) (layer "F.Cu") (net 7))
 (via (at 152.4 91.44) (size 0.8) (drill 0.4) (layers "F.Cu" "B.Cu") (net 7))
 (via (at 154.94 99.06) (size 0.8) (drill 0.4) (layers "F.Cu" "B.Cu") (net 7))
 (segment (start 157.48 96.52) (end 157.48 99.06) (width 0.25) (layer "B.Cu") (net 7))
 (segment (start 152.4 91.44) (end 157.48 96.52) (width 0.25) (layer "B.Cu") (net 7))
 (segment (start 157.48 99.06) (end 154.94 99.06) (width 0.25) (layer "B.Cu") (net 7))
 (segment (start 133.995 95.895) (end 133.995 92.98) (width 0.25) (layer "F.Cu") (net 9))
 (segment (start 143.0425 97.3225) (end 142.24 96.52) (width 0.25) (layer "F.Cu") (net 9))
 (segment (start 134.62 96.52) (end 133.995 95.895) (width 0.25) (layer "F.Cu") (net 9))
 (segment (start 133.62 101.665) (end 133.995 101.29) (width 0.25) (layer "F.Cu") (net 9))
 (segment (start 137.16 96.52) (end 134.62 96.52) (width 0.25) (layer "F.Cu") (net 9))
 (segment (start 133.995 101.29) (end 133.995 95.895) (width 0.25) (layer "F.Cu") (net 9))
 (segment (start 147.385 97.3225) (end 143.0425 97.3225) (width 0.25) (layer "F.Cu") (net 9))
 (via (at 137.16 96.52) (size 0.8) (drill 0.4) (layers "F.Cu" "B.Cu") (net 9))
 (via (at 142.24 96.52) (size 0.8) (drill 0.4) (layers "F.Cu" "B.Cu") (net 9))
 (segment (start 142.24 96.52) (end 137.16 96.52) (width 0.25) (layer "B.Cu") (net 9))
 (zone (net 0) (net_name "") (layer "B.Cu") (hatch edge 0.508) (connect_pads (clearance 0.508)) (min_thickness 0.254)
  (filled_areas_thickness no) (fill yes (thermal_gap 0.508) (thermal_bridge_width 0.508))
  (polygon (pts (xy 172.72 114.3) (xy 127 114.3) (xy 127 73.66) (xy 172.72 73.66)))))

